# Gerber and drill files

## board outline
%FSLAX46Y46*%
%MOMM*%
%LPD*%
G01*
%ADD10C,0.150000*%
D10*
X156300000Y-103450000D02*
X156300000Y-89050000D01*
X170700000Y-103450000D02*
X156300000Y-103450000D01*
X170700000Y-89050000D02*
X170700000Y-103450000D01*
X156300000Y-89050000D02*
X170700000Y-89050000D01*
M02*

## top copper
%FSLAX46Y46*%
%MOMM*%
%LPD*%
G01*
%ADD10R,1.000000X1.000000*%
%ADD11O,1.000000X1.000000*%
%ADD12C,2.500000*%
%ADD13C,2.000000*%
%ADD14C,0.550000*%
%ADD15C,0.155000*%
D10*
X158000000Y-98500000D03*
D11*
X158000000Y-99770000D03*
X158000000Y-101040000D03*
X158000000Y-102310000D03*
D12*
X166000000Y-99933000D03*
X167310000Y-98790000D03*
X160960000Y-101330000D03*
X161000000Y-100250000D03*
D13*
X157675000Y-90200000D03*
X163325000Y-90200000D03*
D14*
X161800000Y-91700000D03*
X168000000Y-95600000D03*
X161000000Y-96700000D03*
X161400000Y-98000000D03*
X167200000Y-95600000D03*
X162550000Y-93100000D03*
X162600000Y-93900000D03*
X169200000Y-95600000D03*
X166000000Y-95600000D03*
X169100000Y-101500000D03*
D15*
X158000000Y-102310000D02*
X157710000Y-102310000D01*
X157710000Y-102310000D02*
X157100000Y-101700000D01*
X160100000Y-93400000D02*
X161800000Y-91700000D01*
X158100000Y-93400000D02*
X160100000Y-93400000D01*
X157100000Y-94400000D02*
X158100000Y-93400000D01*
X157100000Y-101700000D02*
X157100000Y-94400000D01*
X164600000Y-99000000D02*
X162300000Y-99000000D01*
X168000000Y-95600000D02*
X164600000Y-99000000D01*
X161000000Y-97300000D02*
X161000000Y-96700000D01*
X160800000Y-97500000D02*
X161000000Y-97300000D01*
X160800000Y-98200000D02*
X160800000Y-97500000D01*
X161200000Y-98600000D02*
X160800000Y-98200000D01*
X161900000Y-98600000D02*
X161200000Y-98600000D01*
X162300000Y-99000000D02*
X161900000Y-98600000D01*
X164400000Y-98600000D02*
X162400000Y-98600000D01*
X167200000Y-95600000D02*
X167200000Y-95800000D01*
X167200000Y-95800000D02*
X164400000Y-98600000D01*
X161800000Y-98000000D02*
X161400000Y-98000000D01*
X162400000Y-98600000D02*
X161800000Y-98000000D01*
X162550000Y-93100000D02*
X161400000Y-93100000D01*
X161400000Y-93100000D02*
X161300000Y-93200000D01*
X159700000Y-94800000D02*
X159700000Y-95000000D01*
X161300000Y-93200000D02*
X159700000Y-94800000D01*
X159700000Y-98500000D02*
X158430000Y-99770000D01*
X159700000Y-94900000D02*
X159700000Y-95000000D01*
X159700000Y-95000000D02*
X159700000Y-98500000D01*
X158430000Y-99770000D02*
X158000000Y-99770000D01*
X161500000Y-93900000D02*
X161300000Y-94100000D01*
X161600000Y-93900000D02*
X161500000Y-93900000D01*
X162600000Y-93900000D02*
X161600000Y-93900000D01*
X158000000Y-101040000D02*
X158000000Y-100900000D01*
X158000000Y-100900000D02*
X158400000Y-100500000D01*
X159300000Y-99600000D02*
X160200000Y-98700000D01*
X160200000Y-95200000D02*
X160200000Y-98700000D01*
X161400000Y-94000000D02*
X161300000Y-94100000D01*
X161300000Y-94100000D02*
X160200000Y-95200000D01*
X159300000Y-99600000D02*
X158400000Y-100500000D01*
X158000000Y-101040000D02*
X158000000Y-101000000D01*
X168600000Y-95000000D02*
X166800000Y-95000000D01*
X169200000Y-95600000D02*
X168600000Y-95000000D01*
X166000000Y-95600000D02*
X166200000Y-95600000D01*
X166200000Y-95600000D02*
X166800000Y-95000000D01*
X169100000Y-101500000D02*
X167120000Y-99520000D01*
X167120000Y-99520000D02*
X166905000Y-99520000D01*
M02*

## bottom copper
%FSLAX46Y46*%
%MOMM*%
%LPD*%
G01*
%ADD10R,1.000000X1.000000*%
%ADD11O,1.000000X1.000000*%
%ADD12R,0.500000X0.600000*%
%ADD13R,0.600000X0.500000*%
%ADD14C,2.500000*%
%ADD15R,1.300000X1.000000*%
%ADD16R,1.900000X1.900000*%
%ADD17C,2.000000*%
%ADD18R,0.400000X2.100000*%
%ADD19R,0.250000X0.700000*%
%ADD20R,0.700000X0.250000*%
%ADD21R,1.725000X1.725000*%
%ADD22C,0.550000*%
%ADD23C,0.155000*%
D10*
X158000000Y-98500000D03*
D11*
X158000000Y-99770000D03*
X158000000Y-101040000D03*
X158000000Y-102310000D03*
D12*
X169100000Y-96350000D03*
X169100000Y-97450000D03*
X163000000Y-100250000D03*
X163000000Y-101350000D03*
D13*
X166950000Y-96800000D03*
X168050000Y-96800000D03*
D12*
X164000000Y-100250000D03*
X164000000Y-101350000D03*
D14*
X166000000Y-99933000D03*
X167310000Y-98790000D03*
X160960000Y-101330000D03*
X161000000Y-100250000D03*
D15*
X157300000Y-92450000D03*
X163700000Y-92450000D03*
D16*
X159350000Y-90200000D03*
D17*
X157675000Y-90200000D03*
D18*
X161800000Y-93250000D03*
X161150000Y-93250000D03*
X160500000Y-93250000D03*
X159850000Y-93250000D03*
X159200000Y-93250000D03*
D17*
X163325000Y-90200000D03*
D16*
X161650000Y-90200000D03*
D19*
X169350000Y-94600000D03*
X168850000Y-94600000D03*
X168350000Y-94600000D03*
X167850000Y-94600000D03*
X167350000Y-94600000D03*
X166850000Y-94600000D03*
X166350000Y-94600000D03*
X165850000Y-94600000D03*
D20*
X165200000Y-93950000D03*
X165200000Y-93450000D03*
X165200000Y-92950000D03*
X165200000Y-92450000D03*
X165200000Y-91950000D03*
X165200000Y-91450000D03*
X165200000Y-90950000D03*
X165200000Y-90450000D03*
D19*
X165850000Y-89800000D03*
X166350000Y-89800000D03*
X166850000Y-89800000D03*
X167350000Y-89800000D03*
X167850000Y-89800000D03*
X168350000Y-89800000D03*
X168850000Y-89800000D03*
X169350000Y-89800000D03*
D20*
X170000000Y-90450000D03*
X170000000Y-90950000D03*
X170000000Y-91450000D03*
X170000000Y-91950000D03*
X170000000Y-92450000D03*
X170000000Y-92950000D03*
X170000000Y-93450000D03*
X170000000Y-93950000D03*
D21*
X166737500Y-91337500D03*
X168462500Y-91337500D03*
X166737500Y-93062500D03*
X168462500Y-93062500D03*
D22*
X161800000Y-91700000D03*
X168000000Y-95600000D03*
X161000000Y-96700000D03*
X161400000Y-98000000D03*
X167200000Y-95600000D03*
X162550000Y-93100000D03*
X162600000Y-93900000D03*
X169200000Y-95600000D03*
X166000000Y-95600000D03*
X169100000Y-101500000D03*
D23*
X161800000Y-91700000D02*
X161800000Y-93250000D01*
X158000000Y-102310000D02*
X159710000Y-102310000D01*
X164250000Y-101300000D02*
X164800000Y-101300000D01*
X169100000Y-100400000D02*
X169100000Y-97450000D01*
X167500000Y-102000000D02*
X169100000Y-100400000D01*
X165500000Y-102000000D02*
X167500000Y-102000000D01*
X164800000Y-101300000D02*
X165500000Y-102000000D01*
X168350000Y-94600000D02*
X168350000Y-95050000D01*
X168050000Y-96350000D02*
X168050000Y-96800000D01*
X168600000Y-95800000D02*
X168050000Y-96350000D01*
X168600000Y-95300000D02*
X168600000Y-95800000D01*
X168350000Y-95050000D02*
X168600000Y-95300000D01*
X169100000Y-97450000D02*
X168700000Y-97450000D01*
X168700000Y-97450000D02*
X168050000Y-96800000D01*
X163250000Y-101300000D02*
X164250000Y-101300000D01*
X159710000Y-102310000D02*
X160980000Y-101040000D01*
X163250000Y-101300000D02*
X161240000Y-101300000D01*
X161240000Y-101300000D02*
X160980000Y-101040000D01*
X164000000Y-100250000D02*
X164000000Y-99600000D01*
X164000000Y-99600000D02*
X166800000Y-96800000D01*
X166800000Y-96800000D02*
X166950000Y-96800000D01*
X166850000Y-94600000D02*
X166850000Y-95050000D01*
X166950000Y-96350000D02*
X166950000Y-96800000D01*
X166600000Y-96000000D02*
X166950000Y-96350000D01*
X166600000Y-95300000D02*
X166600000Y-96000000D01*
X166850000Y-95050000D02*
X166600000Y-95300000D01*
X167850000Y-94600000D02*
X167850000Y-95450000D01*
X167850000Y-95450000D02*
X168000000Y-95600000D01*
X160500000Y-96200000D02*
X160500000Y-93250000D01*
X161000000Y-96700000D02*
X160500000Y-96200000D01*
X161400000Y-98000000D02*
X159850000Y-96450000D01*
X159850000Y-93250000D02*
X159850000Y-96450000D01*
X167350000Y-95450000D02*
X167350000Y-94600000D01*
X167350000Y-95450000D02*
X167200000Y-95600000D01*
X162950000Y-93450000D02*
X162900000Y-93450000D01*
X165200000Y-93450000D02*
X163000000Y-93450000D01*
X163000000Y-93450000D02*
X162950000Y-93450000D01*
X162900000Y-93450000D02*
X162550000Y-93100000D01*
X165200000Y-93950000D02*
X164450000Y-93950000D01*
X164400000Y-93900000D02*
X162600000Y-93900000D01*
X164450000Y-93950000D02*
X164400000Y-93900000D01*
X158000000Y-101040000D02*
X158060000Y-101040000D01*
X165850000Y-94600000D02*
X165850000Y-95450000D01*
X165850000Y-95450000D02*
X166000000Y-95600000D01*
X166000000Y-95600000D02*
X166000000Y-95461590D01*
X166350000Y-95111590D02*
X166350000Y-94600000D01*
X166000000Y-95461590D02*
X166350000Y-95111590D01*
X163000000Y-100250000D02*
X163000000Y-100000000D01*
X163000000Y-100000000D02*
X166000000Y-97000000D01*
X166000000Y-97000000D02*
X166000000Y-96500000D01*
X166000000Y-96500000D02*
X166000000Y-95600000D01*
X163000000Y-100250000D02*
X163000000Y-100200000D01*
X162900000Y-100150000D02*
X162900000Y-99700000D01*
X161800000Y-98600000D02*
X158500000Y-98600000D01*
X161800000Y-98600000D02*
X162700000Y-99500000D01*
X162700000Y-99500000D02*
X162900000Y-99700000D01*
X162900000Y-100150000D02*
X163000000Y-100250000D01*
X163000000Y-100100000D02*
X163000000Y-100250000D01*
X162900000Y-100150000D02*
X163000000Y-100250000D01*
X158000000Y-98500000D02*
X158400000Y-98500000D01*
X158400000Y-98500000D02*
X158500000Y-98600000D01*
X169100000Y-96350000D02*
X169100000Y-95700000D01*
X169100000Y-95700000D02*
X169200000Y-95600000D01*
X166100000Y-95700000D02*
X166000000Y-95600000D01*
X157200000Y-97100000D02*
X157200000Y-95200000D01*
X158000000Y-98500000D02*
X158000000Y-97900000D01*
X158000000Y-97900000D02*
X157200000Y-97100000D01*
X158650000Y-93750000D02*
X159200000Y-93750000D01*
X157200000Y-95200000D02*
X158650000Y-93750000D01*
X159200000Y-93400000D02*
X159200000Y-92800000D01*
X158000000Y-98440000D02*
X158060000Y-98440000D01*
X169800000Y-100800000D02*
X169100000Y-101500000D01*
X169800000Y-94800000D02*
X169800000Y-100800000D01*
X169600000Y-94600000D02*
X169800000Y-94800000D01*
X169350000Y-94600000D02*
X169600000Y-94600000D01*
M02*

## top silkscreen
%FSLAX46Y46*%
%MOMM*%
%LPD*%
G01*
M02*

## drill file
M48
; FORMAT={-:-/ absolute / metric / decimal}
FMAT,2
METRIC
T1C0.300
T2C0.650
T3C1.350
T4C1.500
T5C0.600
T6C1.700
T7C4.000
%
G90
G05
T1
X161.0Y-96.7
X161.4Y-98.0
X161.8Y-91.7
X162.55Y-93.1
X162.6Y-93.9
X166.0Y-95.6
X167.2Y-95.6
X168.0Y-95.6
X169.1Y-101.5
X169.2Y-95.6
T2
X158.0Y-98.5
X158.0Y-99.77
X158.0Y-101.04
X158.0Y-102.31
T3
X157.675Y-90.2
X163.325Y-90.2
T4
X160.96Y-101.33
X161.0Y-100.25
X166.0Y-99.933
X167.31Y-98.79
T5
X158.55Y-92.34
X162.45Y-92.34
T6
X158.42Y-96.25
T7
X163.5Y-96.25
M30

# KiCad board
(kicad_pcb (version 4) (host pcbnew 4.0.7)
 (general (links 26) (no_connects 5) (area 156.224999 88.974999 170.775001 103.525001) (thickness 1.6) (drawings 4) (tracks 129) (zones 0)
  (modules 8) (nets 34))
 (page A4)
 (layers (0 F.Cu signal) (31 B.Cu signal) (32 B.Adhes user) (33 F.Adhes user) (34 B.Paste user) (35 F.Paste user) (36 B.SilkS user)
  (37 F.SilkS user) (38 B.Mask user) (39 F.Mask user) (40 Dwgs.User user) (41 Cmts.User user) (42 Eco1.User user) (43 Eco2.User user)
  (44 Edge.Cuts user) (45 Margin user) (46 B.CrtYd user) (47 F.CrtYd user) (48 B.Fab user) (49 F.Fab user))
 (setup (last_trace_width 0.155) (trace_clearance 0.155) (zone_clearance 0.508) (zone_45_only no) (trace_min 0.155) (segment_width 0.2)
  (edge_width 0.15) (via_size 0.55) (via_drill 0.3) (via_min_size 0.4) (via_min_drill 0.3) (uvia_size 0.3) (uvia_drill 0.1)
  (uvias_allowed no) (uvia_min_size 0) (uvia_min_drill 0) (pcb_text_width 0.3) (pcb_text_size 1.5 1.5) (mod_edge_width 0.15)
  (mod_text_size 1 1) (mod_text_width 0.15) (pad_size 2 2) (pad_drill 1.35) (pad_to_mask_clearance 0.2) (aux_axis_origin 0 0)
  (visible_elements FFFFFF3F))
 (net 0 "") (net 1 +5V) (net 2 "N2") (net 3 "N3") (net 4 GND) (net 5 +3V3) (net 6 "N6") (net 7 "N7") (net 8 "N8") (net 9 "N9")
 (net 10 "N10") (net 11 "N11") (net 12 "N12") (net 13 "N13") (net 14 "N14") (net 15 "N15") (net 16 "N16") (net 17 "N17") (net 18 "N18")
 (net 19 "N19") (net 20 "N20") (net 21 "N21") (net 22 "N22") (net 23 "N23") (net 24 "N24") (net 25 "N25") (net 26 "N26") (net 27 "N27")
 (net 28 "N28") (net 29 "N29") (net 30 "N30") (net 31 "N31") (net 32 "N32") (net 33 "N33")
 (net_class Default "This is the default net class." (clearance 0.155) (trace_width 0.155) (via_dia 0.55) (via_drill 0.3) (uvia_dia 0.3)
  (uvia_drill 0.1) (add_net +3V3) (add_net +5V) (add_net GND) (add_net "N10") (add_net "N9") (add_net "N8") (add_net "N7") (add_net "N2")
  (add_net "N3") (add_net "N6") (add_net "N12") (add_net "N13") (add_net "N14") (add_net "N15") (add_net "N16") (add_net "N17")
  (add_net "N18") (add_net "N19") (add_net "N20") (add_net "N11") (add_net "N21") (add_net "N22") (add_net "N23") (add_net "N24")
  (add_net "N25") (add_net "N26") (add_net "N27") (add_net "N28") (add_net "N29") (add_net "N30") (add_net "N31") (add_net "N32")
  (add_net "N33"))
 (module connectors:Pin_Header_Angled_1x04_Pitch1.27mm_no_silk (layer B.Cu) (at 158 98.5 180)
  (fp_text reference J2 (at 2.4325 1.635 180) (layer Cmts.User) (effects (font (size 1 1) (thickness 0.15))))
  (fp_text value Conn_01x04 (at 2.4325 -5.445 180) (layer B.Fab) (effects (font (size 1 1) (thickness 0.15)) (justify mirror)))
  (pad 1 thru_hole rect (at 0 0 180) (size 1 1) (drill 0.65) (layers *.Cu *.Mask) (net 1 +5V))
  (pad 2 thru_hole oval (at 0 -1.27 180) (size 1 1) (drill 0.65) (layers *.Cu *.Mask) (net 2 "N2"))
  (pad 3 thru_hole oval (at 0 -2.54 180) (size 1 1) (drill 0.65) (layers *.Cu *.Mask) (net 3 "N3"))
  (pad 4 thru_hole oval (at 0 -3.81 180) (size 1 1) (drill 0.65) (layers *.Cu *.Mask) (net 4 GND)))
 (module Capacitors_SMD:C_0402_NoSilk (layer B.Cu) (at 169.1 96.9 270)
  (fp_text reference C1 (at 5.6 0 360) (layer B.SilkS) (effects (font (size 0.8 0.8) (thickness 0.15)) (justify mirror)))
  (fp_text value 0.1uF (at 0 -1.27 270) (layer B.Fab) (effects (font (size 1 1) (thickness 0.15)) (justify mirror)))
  (pad 1 smd rect (at -0.55 0 270) (size 0.6 0.5) (layers B.Cu B.Paste B.Mask) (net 1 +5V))
  (pad 2 smd rect (at 0.55 0 270) (size 0.6 0.5) (layers B.Cu B.Paste B.Mask) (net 4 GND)))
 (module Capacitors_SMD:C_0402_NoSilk (layer B.Cu) (at 163 100.8 270)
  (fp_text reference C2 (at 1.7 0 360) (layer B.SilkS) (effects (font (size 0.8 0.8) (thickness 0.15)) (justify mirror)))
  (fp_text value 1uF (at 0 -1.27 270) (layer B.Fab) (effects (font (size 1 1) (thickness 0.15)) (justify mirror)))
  (pad 1 smd rect (at -0.55 0 270) (size 0.6 0.5) (layers B.Cu B.Paste B.Mask) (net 1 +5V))
  (pad 2 smd rect (at 0.55 0 270) (size 0.6 0.5) (layers B.Cu B.Paste B.Mask) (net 4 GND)))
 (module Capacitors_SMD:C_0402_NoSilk (layer B.Cu) (at 167.5 96.8)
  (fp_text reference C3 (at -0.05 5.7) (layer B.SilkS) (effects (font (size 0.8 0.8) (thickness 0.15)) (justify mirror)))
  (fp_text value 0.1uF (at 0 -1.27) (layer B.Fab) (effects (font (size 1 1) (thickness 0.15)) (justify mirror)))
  (pad 1 smd rect (at -0.55 0) (size 0.6 0.5) (layers B.Cu B.Paste B.Mask) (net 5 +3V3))
  (pad 2 smd rect (at 0.55 0) (size 0.6 0.5) (layers B.Cu B.Paste B.Mask) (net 4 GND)))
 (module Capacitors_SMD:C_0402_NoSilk (layer B.Cu) (at 164 100.8 270)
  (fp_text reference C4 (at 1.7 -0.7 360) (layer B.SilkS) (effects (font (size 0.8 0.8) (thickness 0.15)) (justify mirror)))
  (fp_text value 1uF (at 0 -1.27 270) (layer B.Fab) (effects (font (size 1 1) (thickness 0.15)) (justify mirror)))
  (pad 1 smd rect (at -0.55 0 270) (size 0.6 0.5) (layers B.Cu B.Paste B.Mask) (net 5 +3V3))
  (pad 2 smd rect (at 0.55 0 270) (size 0.6 0.5) (layers B.Cu B.Paste B.Mask) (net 4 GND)))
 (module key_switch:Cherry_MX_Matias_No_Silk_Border (layer B.Cu) (at 163.5 96.25)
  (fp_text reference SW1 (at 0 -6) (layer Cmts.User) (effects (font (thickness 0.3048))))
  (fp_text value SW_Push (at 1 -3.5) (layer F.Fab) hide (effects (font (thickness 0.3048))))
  (pad 2 thru_hole circle (at 2.5 3.683) (size 2.5 2.5) (drill 1.5) (layers *.Cu *.Mask) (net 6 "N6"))
  (pad 2 thru_hole circle (at 3.81 2.54) (size 2.5 2.5) (drill 1.5) (layers *.Cu *.Mask) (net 6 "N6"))
  (pad "" np_thru_hole circle (at 0 0) (size 4 4) (drill 4) (layers *.Cu *.Mask B.SilkS))
  (pad "" np_thru_hole circle (at -5.08 0) (size 1.7 1.7) (drill 1.7) (layers *.Cu *.Mask B.SilkS))
  (pad 1 thru_hole circle (at -2.54 5.08) (size 2.5 2.5) (drill 1.5) (layers *.Cu *.Mask) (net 4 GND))
  (pad 1 thru_hole circle (at -2.5 4) (size 2.5 2.5) (drill 1.5) (layers *.Cu *.Mask) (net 4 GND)))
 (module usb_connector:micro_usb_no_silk (layer B.Cu) (at 160.5 92.2)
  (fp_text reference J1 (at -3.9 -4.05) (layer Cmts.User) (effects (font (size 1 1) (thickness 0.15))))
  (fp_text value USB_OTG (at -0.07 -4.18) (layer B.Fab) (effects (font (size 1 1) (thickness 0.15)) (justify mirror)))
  (pad 6 smd rect (at -3.2 0.25) (size 1.3 1) (layers B.Cu B.Paste B.Mask) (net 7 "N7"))
  (pad 6 smd rect (at 3.2 0.25) (size 1.3 1) (layers B.Cu B.Paste B.Mask) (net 7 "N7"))
  (pad "" np_thru_hole circle (at -1.95 0.14) (size 0.6 0.6) (drill 0.6) (layers *.Cu *.Mask))
  (pad 6 smd rect (at -1.15 -2) (size 1.9 1.9) (layers B.Cu B.Paste B.Mask) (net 7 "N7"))
  (pad 6 thru_hole circle (at -2.825 -2) (size 2 2) (drill 1.35) (layers *.Cu *.Mask) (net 7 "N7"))
  (pad 5 smd rect (at 1.3 1.05) (size 0.4 2.1) (layers B.Cu B.Paste B.Mask) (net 4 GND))
  (pad 4 smd rect (at 0.65 1.05) (size 0.4 2.1) (layers B.Cu B.Paste B.Mask) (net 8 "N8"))
  (pad 3 smd rect (at 0 1.05) (size 0.4 2.1) (layers B.Cu B.Paste B.Mask) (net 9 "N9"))
  (pad 2 smd rect (at -0.65 1.05) (size 0.4 2.1) (layers B.Cu B.Paste B.Mask) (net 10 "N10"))
  (pad 1 smd rect (at -1.3 1.05) (size 0.4 2.1) (layers B.Cu B.Paste B.Mask) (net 1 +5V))
  (pad 6 thru_hole circle (at 2.825 -2) (size 2 2) (drill 1.35) (layers *.Cu *.Mask) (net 7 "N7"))
  (pad 6 smd rect (at 1.15 -2) (size 1.9 1.9) (layers B.Cu B.Paste B.Mask) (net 7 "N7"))
  (pad "" np_thru_hole circle (at 1.95 0.14) (size 0.6 0.6) (drill 0.6) (layers *.Cu *.Mask)))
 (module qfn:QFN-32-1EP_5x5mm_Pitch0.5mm (layer B.Cu) (at 167.6 92.2 90)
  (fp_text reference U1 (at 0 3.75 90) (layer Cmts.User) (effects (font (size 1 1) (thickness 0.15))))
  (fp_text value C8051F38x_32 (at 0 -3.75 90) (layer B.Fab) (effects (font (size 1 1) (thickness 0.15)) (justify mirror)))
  (pad 1 smd rect (at -2.4 1.75 90) (size 0.7 0.25) (layers B.Cu B.Paste B.Mask) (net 6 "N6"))
  (pad 2 smd rect (at -2.4 1.25 90) (size 0.7 0.25) (layers B.Cu B.Paste B.Mask) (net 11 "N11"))
  (pad 3 smd rect (at -2.4 0.75 90) (size 0.7 0.25) (layers B.Cu B.Paste B.Mask) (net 4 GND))
  (pad 4 smd rect (at -2.4 0.25 90) (size 0.7 0.25) (layers B.Cu B.Paste B.Mask) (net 9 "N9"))
  (pad 5 smd rect (at -2.4 -0.25 90) (size 0.7 0.25) (layers B.Cu B.Paste B.Mask) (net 10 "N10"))
  (pad 6 smd rect (at -2.4 -0.75 90) (size 0.7 0.25) (layers B.Cu B.Paste B.Mask) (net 5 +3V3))
  (pad 7 smd rect (at -2.4 -1.25 90) (size 0.7 0.25) (layers B.Cu B.Paste B.Mask) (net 1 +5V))
  (pad 8 smd rect (at -2.4 -1.75 90) (size 0.7 0.25) (layers B.Cu B.Paste B.Mask) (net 1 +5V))
  (pad 9 smd rect (at -1.75 -2.4) (size 0.7 0.25) (layers B.Cu B.Paste B.Mask) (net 3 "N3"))
  (pad 10 smd rect (at -1.25 -2.4) (size 0.7 0.25) (layers B.Cu B.Paste B.Mask) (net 2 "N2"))
  (pad 11 smd rect (at -0.75 -2.4) (size 0.7 0.25) (layers B.Cu B.Paste B.Mask) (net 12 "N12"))
  (pad 12 smd rect (at -0.25 -2.4) (size 0.7 0.25) (layers B.Cu B.Paste B.Mask) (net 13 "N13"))
  (pad 13 smd rect (at 0.25 -2.4) (size 0.7 0.25) (layers B.Cu B.Paste B.Mask) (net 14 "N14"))
  (pad 14 smd rect (at 0.75 -2.4) (size 0.7 0.25) (layers B.Cu B.Paste B.Mask) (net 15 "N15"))
  (pad 15 smd rect (at 1.25 -2.4) (size 0.7 0.25) (layers B.Cu B.Paste B.Mask) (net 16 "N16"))
  (pad 16 smd rect (at 1.75 -2.4) (size 0.7 0.25) (layers B.Cu B.Paste B.Mask) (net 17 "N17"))
  (pad 17 smd rect (at 2.4 -1.75 90) (size 0.7 0.25) (layers B.Cu B.Paste B.Mask) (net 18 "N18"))
  (pad 18 smd rect (at 2.4 -1.25 90) (size 0.7 0.25) (layers B.Cu B.Paste B.Mask) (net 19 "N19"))
  (pad 19 smd rect (at 2.4 -0.75 90) (size 0.7 0.25) (layers B.Cu B.Paste B.Mask) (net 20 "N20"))
  (pad 20 smd rect (at 2.4 -0.25 90) (size 0.7 0.25) (layers B.Cu B.Paste B.Mask) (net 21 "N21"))
  (pad 21 smd rect (at 2.4 0.25 90) (size 0.7 0.25) (layers B.Cu B.Paste B.Mask) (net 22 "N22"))
  (pad 22 smd rect (at 2.4 0.75 90) (size 0.7 0.25) (layers B.Cu B.Paste B.Mask) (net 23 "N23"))
  (pad 23 smd rect (at 2.4 1.25 90) (size 0.7 0.25) (layers B.Cu B.Paste B.Mask) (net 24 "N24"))
  (pad 24 smd rect (at 2.4 1.75 90) (size 0.7 0.25) (layers B.Cu B.Paste B.Mask) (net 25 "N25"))
  (pad 25 smd rect (at 1.75 2.4) (size 0.7 0.25) (layers B.Cu B.Paste B.Mask) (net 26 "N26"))
  (pad 26 smd rect (at 1.25 2.4) (size 0.7 0.25) (layers B.Cu B.Paste B.Mask) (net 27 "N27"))
  (pad 27 smd rect (at 0.75 2.4) (size 0.7 0.25) (layers B.Cu B.Paste B.Mask) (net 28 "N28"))
  (pad 28 smd rect (at 0.25 2.4) (size 0.7 0.25) (layers B.Cu B.Paste B.Mask) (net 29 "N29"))
  (pad 29 smd rect (at -0.25 2.4) (size 0.7 0.25) (layers B.Cu B.Paste B.Mask) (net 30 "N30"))
  (pad 30 smd rect (at -0.75 2.4) (size 0.7 0.25) (layers B.Cu B.Paste B.Mask) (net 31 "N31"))
  (pad 31 smd rect (at -1.25 2.4) (size 0.7 0.25) (layers B.Cu B.Paste B.Mask) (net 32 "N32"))
  (pad 32 smd rect (at -1.75 2.4) (size 0.7 0.25) (layers B.Cu B.Paste B.Mask) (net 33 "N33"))
  (pad 33 smd rect (at 0.8625 -0.8625 90) (size 1.725 1.725) (layers B.Cu B.Paste B.Mask) (solder_paste_margin_ratio -0.2))
  (pad 33 smd rect (at 0.8625 0.8625 90) (size 1.725 1.725) (layers B.Cu B.Paste B.Mask) (solder_paste_margin_ratio -0.2))
  (pad 33 smd rect (at -0.8625 -0.8625 90) (size 1.725 1.725) (layers B.Cu B.Paste B.Mask) (solder_paste_margin_ratio -0.2))
  (pad 33 smd rect (at -0.8625 0.8625 90) (size 1.725 1.725) (layers B.Cu B.Paste B.Mask) (solder_paste_margin_ratio -0.2)))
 (gr_line (start 156.3 103.45) (end 156.3 89.05) (angle 90) (layer Edge.Cuts) (width 0.15))
 (gr_line (start 170.7 103.45) (end 156.3 103.45) (angle 90) (layer Edge.Cuts) (width 0.15))
 (gr_line (start 170.7 89.05) (end 170.7 103.45) (angle 90) (layer Edge.Cuts) (width 0.15))
 (gr_line (start 156.3 89.05) (end 170.7 89.05) (angle 90) (layer Edge.Cuts) (width 0.15))
 (segment (start 158 102.31) (end 157.71 102.31) (width 0.155) (layer F.Cu) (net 4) (status 30))
 (segment (start 157.71 102.31) (end 157.1 101.7) (width 0.155) (layer F.Cu) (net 4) (status 10))
 (segment (start 161.8 91.7) (end 161.8 93.25) (width 0.155) (layer B.Cu) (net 4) (status 20))
 (via (at 161.8 91.7) (size 0.55) (drill 0.3) (layers F.Cu B.Cu) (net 4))
 (segment (start 160.1 93.4) (end 161.8 91.7) (width 0.155) (layer F.Cu) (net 4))
 (segment (start 158.1 93.4) (end 160.1 93.4) (width 0.155) (layer F.Cu) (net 4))
 (segment (start 157.1 94.4) (end 158.1 93.4) (width 0.155) (layer F.Cu) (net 4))
 (segment (start 157.1 101.7) (end 157.1 94.4) (width 0.155) (layer F.Cu) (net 4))
 (segment (start 158 102.31) (end 159.71 102.31) (width 0.155) (layer B.Cu) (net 4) (status 10))
 (segment (start 164.25 101.3) (end 164.8 101.3) (width 0.155) (layer B.Cu) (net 4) (status 10))
 (segment (start 169.1 100.4) (end 169.1 97.45) (width 0.155) (layer B.Cu) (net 4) (status 20))
 (segment (start 167.5 102) (end 169.1 100.4) (width 0.155) (layer B.Cu) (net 4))
 (segment (start 165.5 102) (end 167.5 102) (width 0.155) (layer B.Cu) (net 4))
 (segment (start 164.8 101.3) (end 165.5 102) (width 0.155) (layer B.Cu) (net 4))
 (segment (start 168.35 94.6) (end 168.35 95.05) (width 0.155) (layer B.Cu) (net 4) (status 10))
 (segment (start 168.05 96.35) (end 168.05 96.8) (width 0.155) (layer B.Cu) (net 4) (status 20))
 (segment (start 168.6 95.8) (end 168.05 96.35) (width 0.155) (layer B.Cu) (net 4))
 (segment (start 168.6 95.3) (end 168.6 95.8) (width 0.155) (layer B.Cu) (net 4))
 (segment (start 168.35 95.05) (end 168.6 95.3) (width 0.155) (layer B.Cu) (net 4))
 (segment (start 169.1 97.45) (end 168.7 97.45) (width 0.155) (layer B.Cu) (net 4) (status 10))
 (segment (start 168.7 97.45) (end 168.05 96.8) (width 0.155) (layer B.Cu) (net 4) (status 20))
 (segment (start 163.25 101.3) (end 164.25 101.3) (width 0.155) (layer B.Cu) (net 4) (status 30))
 (segment (start 159.71 102.31) (end 160.98 101.04) (width 0.155) (layer B.Cu) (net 4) (status 20))
 (segment (start 163.25 101.3) (end 161.24 101.3) (width 0.155) (layer B.Cu) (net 4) (status 30))
 (segment (start 161.24 101.3) (end 160.98 101.04) (width 0.155) (layer B.Cu) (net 4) (status 30))
 (segment (start 164 100.25) (end 164 99.6) (width 0.155) (layer B.Cu) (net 5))
 (segment (start 164 99.6) (end 166.8 96.8) (width 0.155) (layer B.Cu) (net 5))
 (segment (start 166.8 96.8) (end 166.95 96.8) (width 0.155) (layer B.Cu) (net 5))
 (segment (start 166.85 94.6) (end 166.85 95.05) (width 0.155) (layer B.Cu) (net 5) (status 10))
 (segment (start 166.95 96.35) (end 166.95 96.8) (width 0.155) (layer B.Cu) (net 5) (status 20))
 (segment (start 166.6 96) (end 166.95 96.35) (width 0.155) (layer B.Cu) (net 5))
 (segment (start 166.6 95.3) (end 166.6 96) (width 0.155) (layer B.Cu) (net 5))
 (segment (start 166.85 95.05) (end 166.6 95.3) (width 0.155) (layer B.Cu) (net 5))
 (segment (start 164.6 99) (end 162.3 99) (width 0.155) (layer F.Cu) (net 9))
 (segment (start 167.85 94.6) (end 167.85 95.45) (width 0.155) (layer B.Cu) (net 9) (status 10))
 (segment (start 168 95.6) (end 164.6 99) (width 0.155) (layer F.Cu) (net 9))
 (via (at 168 95.6) (size 0.55) (drill 0.3) (layers F.Cu B.Cu) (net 9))
 (segment (start 167.85 95.45) (end 168 95.6) (width 0.155) (layer B.Cu) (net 9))
 (segment (start 161 97.3) (end 161 96.7) (width 0.155) (layer F.Cu) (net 9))
 (segment (start 160.8 97.5) (end 161 97.3) (width 0.155) (layer F.Cu) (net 9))
 (segment (start 160.8 98.2) (end 160.8 97.5) (width 0.155) (layer F.Cu) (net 9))
 (segment (start 161.2 98.6) (end 160.8 98.2) (width 0.155) (layer F.Cu) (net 9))
 (segment (start 161.9 98.6) (end 161.2 98.6) (width 0.155) (layer F.Cu) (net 9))
 (segment (start 162.3 99) (end 161.9 98.6) (width 0.155) (layer F.Cu) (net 9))
 (segment (start 160.5 96.2) (end 160.5 93.25) (width 0.155) (layer B.Cu) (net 9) (status 20))
 (segment (start 161 96.7) (end 160.5 96.2) (width 0.155) (layer B.Cu) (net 9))
 (via (at 161 96.7) (size 0.55) (drill 0.3) (layers F.Cu B.Cu) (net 9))
 (segment (start 164.4 98.6) (end 162.4 98.6) (width 0.155) (layer F.Cu) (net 10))
 (via (at 161.4 98) (size 0.55) (drill 0.3) (layers F.Cu B.Cu) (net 10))
 (segment (start 161.4 98) (end 159.85 96.45) (width 0.155) (layer B.Cu) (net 10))
 (segment (start 159.85 93.25) (end 159.85 96.45) (width 0.155) (layer B.Cu) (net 10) (status 20))
 (segment (start 167.2 95.6) (end 167.2 95.8) (width 0.155) (layer F.Cu) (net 10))
 (segment (start 167.2 95.8) (end 164.4 98.6) (width 0.155) (layer F.Cu) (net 10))
 (segment (start 167.35 95.45) (end 167.35 94.6) (width 0.155) (layer B.Cu) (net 10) (status 10))
 (via (at 167.2 95.6) (size 0.55) (drill 0.3) (layers F.Cu B.Cu) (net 10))
 (segment (start 167.35 95.45) (end 167.2 95.6) (width 0.155) (layer B.Cu) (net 10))
 (segment (start 161.8 98) (end 161.4 98) (width 0.155) (layer F.Cu) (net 10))
 (segment (start 162.4 98.6) (end 161.8 98) (width 0.155) (layer F.Cu) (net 10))
 (segment (start 162.95 93.45) (end 162.9 93.45) (width 0.155) (layer B.Cu) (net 2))
 (segment (start 165.2 93.45) (end 163 93.45) (width 0.155) (layer B.Cu) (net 2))
 (via (at 162.55 93.1) (size 0.55) (drill 0.3) (layers F.Cu B.Cu) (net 2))
 (segment (start 162.55 93.1) (end 161.4 93.1) (width 0.155) (layer F.Cu) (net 2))
 (segment (start 161.4 93.1) (end 161.3 93.2) (width 0.155) (layer F.Cu) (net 2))
 (segment (start 159.7 94.8) (end 159.7 95) (width 0.155) (layer F.Cu) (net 2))
 (segment (start 161.3 93.2) (end 159.7 94.8) (width 0.155) (layer F.Cu) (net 2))
 (segment (start 163 93.45) (end 162.95 93.45) (width 0.155) (layer B.Cu) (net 2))
 (segment (start 162.9 93.45) (end 162.55 93.1) (width 0.155) (layer B.Cu) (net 2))
 (segment (start 159.7 98.5) (end 158.43 99.77) (width 0.155) (layer F.Cu) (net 2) (status 20))
 (segment (start 159.7 94.9) (end 159.7 95) (width 0.155) (layer F.Cu) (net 2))
 (segment (start 159.7 95) (end 159.7 98.5) (width 0.155) (layer F.Cu) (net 2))
 (segment (start 158.43 99.77) (end 158 99.77) (width 0.155) (layer F.Cu) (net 2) (status 30))
 (segment (start 165.2 93.95) (end 164.45 93.95) (width 0.155) (layer B.Cu) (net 3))
 (segment (start 161.5 93.9) (end 161.3 94.1) (width 0.155) (layer F.Cu) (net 3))
 (segment (start 161.6 93.9) (end 161.5 93.9) (width 0.155) (layer F.Cu) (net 3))
 (segment (start 162.6 93.9) (end 161.6 93.9) (width 0.155) (layer F.Cu) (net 3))
 (via (at 162.6 93.9) (size 0.55) (drill 0.3) (layers F.Cu B.Cu) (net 3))
 (segment (start 164.4 93.9) (end 162.6 93.9) (width 0.155) (layer B.Cu) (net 3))
 (segment (start 164.45 93.95) (end 164.4 93.9) (width 0.155) (layer B.Cu) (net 3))
 (segment (start 158 101.04) (end 158 100.9) (width 0.155) (layer F.Cu) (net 3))
 (segment (start 158 100.9) (end 158.4 100.5) (width 0.155) (layer F.Cu) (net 3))
 (segment (start 159.3 99.6) (end 160.2 98.7) (width 0.155) (layer F.Cu) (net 3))
 (segment (start 160.2 95.2) (end 160.2 98.7) (width 0.155) (layer F.Cu) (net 3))
 (segment (start 161.4 94) (end 161.3 94.1) (width 0.155) (layer F.Cu) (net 3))
 (segment (start 161.3 94.1) (end 160.2 95.2) (width 0.155) (layer F.Cu) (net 3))
 (segment (start 159.3 99.6) (end 158.4 100.5) (width 0.155) (layer F.Cu) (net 3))
 (segment (start 158 101.04) (end 158 101) (width 0.155) (layer F.Cu) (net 3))
 (segment (start 158 101.04) (end 158.06 101.04) (width 0.155) (layer B.Cu) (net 3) (status 30))
 (segment (start 165.85 94.6) (end 165.85 95.45) (width 0.155) (layer B.Cu) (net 1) (status 400000))
 (segment (start 165.85 95.45) (end 166 95.6) (width 0.155) (layer B.Cu) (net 1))
 (segment (start 166 95.6) (end 166 95.46159) (width 0.155) (layer B.Cu) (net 1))
 (segment (start 166.35 95.11159) (end 166.35 94.6) (width 0.155) (layer B.Cu) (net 1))
 (segment (start 166 95.46159) (end 166.35 95.11159) (width 0.155) (layer B.Cu) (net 1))
 (segment (start 163 100.25) (end 163 100) (width 0.155) (layer B.Cu) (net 1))
 (segment (start 163 100) (end 166 97) (width 0.155) (layer B.Cu) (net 1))
 (segment (start 166 97) (end 166 96.5) (width 0.155) (layer B.Cu) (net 1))
 (segment (start 166 96.5) (end 166 95.6) (width 0.155) (layer B.Cu) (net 1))
 (segment (start 163 100.25) (end 163 100.2) (width 0.155) (layer B.Cu) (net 1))
 (segment (start 162.9 100.15) (end 162.9 99.7) (width 0.155) (layer B.Cu) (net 1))
 (segment (start 161.8 98.6) (end 158.5 98.6) (width 0.155) (layer B.Cu) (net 1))
 (segment (start 161.8 98.6) (end 162.7 99.5) (width 0.155) (layer B.Cu) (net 1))
 (segment (start 162.7 99.5) (end 162.9 99.7) (width 0.155) (layer B.Cu) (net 1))
 (segment (start 162.9 100.15) (end 163 100.25) (width 0.155) (layer B.Cu) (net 1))
 (segment (start 163 100.1) (end 163 100.25) (width 0.155) (layer B.Cu) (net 1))
 (segment (start 162.9 100.15) (end 163 100.25) (width 0.155) (layer B.Cu) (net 1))
 (segment (start 158 98.5) (end 158.4 98.5) (width 0.155) (layer B.Cu) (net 1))
 (segment (start 158.4 98.5) (end 158.5 98.6) (width 0.155) (layer B.Cu) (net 1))
 (segment (start 169.1 96.35) (end 169.1 95.7) (width 0.155) (layer B.Cu) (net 1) (status 10))
 (segment (start 168.6 95) (end 166.8 95) (width 0.155) (layer F.Cu) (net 1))
 (segment (start 169.2 95.6) (end 168.6 95) (width 0.155) (layer F.Cu) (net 1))
 (via (at 169.2 95.6) (size 0.55) (drill 0.3) (layers F.Cu B.Cu) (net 1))
 (segment (start 169.1 95.7) (end 169.2 95.6) (width 0.155) (layer B.Cu) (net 1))
 (segment (start 166 95.6) (end 166.2 95.6) (width 0.155) (layer F.Cu) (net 1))
 (segment (start 166.1 95.7) (end 166 95.6) (width 0.155) (layer B.Cu) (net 1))
 (via (at 166 95.6) (size 0.55) (drill 0.3) (layers F.Cu B.Cu) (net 1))
 (segment (start 166.2 95.6) (end 166.8 95) (width 0.155) (layer F.Cu) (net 1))
 (segment (start 157.2 97.1) (end 157.2 95.2) (width 0.155) (layer B.Cu) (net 1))
 (segment (start 158 98.5) (end 158 97.9) (width 0.155) (layer B.Cu) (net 1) (status 10))
 (segment (start 158 97.9) (end 157.2 97.1) (width 0.155) (layer B.Cu) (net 1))
 (segment (start 158.65 93.75) (end 159.2 93.75) (width 0.155) (layer B.Cu) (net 1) (status 20))
 (segment (start 157.2 95.2) (end 158.65 93.75) (width 0.155) (layer B.Cu) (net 1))
 (segment (start 159.2 93.4) (end 159.2 92.8) (width 0.155) (layer B.Cu) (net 1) (status 30))
 (segment (start 158 98.44) (end 158.06 98.44) (width 0.155) (layer B.Cu) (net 1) (status 30))
 (segment (start 169.1 101.5) (end 167.12 99.52) (width 0.155) (layer F.Cu) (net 6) (status 20))
 (via (at 169.1 101.5) (size 0.55) (drill 0.3) (layers F.Cu B.Cu) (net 6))
 (segment (start 169.8 100.8) (end 169.1 101.5) (width 0.155) (layer B.Cu) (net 6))
 (segment (start 169.8 94.8) (end 169.8 100.8) (width 0.155) (layer B.Cu) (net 6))
 (segment (start 167.12 99.52) (end 166.905 99.52) (width 0.155) (layer F.Cu) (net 6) (status 30))
 (segment (start 169.6 94.6) (end 169.8 94.8) (width 0.155) (layer B.Cu) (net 6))
 (segment (start 169.35 94.6) (end 169.6 94.6) (width 0.155) (layer B.Cu) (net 6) (status 10)))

